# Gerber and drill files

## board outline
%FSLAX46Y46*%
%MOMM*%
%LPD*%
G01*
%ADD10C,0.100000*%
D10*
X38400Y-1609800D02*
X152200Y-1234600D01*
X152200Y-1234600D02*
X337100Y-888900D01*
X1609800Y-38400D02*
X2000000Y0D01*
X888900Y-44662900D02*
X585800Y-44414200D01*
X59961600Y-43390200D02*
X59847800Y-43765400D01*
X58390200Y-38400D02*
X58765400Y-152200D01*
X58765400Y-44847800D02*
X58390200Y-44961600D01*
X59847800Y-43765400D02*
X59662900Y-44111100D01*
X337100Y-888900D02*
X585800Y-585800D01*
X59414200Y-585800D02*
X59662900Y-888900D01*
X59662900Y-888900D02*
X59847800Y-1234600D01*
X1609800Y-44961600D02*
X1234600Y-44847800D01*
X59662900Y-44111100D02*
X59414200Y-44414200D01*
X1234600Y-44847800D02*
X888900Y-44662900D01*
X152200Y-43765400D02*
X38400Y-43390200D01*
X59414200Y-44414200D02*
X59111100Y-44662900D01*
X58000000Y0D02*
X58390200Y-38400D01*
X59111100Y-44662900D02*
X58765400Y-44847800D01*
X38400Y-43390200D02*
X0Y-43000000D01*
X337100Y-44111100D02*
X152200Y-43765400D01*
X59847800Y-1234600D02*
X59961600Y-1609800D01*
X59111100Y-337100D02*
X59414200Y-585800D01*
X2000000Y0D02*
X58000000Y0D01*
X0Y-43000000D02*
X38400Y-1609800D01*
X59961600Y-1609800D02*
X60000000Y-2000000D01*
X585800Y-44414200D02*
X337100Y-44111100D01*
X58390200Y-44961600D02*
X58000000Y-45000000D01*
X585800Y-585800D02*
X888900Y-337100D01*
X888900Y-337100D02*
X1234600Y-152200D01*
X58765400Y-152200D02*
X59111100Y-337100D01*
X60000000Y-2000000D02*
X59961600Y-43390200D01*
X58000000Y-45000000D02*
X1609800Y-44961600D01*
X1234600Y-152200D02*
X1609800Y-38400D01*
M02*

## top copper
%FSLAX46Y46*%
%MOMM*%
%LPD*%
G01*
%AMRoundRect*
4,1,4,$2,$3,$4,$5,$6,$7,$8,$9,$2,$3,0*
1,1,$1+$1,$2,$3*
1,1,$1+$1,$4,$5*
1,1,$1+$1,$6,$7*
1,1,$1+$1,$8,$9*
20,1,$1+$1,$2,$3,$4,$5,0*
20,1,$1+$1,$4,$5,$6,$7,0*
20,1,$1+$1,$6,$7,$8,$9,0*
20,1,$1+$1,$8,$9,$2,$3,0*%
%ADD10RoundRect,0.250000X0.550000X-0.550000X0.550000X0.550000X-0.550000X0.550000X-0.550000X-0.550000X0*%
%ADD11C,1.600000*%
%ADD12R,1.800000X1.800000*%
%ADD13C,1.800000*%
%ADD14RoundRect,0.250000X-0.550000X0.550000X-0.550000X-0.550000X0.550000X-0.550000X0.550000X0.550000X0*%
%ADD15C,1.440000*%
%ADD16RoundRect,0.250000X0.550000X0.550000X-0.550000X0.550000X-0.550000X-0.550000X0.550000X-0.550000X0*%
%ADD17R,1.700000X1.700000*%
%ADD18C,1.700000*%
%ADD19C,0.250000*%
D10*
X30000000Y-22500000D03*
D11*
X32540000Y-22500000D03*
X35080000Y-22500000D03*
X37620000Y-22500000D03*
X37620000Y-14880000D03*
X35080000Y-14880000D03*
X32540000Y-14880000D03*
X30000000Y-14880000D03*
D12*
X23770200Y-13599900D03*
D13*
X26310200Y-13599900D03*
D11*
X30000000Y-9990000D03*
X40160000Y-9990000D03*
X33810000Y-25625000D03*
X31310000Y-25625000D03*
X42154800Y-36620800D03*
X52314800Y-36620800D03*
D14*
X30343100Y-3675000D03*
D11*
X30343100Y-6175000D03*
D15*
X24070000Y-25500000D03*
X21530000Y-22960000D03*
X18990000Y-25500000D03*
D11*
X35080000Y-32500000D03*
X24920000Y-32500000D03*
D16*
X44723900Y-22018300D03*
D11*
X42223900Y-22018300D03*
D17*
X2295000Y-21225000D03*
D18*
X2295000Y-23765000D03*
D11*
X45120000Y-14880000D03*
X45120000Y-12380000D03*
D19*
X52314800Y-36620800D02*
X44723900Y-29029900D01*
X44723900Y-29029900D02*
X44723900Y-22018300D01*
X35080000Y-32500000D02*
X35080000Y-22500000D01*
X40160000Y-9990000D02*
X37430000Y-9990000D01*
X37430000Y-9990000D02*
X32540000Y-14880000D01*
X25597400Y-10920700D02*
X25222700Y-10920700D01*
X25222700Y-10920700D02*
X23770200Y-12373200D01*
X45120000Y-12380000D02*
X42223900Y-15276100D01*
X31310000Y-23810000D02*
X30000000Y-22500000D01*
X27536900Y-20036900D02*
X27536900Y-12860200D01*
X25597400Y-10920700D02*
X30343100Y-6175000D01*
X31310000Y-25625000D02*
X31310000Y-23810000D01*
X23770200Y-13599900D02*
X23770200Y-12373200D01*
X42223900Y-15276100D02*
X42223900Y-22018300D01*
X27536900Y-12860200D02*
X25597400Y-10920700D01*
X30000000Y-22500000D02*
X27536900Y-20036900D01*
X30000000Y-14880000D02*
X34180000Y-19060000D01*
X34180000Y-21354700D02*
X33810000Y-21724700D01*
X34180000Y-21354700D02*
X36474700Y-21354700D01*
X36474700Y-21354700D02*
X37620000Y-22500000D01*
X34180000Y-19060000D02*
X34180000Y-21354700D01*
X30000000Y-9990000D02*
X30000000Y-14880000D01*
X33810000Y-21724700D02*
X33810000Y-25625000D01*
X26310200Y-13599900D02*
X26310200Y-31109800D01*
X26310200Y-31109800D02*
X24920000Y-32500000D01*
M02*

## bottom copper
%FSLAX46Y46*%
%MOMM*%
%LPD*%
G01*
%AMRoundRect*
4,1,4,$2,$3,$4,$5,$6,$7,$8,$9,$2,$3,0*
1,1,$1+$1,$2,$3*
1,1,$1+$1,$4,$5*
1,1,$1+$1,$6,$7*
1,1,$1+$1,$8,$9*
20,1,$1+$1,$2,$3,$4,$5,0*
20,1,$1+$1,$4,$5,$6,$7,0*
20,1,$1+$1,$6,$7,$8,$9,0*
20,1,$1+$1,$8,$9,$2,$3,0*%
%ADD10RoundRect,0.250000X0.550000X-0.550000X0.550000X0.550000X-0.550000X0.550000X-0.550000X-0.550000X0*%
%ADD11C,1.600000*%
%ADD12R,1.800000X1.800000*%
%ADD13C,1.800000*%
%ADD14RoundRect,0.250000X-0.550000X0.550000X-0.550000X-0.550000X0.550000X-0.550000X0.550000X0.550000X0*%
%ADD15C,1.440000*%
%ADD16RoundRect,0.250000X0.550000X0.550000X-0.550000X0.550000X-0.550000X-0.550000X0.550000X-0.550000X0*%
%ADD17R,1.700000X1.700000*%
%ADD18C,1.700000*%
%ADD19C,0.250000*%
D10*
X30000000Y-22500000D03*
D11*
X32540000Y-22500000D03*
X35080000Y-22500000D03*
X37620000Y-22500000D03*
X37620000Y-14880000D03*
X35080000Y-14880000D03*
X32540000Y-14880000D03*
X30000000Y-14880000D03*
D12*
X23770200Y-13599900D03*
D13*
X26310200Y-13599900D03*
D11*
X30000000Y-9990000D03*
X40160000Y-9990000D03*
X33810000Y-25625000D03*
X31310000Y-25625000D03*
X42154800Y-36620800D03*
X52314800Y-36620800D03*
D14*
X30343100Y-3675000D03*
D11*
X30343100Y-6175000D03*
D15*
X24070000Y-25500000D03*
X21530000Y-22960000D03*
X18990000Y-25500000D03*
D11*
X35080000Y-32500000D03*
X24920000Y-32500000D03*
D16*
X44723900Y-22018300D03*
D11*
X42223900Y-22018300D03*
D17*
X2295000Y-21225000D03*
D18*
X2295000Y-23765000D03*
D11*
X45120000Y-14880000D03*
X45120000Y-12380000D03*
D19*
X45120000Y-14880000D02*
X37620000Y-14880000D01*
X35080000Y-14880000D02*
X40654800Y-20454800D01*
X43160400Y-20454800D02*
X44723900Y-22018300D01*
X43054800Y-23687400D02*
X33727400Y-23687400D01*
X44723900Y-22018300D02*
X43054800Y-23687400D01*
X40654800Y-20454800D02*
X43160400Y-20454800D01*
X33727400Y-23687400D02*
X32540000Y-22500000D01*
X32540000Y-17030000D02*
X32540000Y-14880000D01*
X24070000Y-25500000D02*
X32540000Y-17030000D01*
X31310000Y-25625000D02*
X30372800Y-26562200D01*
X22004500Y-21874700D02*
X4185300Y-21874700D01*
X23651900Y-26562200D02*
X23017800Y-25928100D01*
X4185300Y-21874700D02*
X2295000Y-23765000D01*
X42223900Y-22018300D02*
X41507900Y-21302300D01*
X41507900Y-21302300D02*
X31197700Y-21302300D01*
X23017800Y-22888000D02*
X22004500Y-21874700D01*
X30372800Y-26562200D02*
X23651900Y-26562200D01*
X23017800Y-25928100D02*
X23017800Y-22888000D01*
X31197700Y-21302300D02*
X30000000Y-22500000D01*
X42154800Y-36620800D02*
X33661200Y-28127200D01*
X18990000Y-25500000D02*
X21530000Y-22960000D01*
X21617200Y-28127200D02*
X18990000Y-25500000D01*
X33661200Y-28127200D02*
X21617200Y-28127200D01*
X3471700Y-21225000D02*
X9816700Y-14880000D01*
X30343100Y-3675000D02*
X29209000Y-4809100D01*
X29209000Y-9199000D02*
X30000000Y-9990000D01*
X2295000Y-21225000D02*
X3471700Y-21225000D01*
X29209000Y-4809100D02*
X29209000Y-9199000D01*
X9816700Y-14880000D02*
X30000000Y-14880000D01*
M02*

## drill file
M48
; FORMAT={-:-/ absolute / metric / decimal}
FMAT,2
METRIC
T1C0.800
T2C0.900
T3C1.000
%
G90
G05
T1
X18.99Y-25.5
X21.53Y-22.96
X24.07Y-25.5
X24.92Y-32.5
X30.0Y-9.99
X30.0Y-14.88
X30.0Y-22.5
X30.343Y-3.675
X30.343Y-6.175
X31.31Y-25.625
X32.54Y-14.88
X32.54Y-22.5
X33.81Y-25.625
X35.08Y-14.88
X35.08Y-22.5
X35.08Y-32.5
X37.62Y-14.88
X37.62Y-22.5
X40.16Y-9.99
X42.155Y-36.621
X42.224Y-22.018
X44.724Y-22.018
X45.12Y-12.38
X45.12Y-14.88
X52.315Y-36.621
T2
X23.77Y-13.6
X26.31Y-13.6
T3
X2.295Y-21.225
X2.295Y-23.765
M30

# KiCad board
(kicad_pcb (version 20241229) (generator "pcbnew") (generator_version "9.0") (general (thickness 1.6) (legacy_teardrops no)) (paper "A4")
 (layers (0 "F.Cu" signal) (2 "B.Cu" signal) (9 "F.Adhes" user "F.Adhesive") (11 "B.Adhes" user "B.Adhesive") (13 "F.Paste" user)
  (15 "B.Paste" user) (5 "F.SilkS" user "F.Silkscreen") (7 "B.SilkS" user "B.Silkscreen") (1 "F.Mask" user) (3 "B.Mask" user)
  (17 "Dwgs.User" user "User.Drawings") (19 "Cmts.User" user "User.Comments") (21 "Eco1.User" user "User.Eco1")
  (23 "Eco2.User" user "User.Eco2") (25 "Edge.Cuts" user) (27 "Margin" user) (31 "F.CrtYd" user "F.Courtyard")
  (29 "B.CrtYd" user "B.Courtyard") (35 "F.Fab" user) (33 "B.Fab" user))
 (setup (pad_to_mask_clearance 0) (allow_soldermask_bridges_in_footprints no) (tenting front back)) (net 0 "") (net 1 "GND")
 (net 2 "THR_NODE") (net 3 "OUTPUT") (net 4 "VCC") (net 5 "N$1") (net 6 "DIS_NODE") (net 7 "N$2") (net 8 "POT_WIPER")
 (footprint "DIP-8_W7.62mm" (layer "F.Cu") (at 30 22.5 90)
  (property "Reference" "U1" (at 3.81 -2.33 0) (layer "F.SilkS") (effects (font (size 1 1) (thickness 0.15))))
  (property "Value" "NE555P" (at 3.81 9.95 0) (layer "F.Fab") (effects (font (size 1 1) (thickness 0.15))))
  (pad "1" thru_hole roundrect (at 0 0 90) (size 1.6 1.6) (drill 0.8) (layers "*.Cu" "*.Mask") (remove_unused_layers no)
   (roundrect_rratio 0.15625) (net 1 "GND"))
  (pad "2" thru_hole circle (at 0 2.54 90) (size 1.6 1.6) (drill 0.8) (layers "*.Cu" "*.Mask") (remove_unused_layers no) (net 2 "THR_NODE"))
  (pad "3" thru_hole circle (at 0 5.08 90) (size 1.6 1.6) (drill 0.8) (layers "*.Cu" "*.Mask") (remove_unused_layers no) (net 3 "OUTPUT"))
  (pad "4" thru_hole circle (at 0 7.62 90) (size 1.6 1.6) (drill 0.8) (layers "*.Cu" "*.Mask") (remove_unused_layers no) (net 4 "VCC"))
  (pad "5" thru_hole circle (at 7.62 7.62 90) (size 1.6 1.6) (drill 0.8) (layers "*.Cu" "*.Mask") (remove_unused_layers no) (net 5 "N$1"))
  (pad "6" thru_hole circle (at 7.62 5.08 90) (size 1.6 1.6) (drill 0.8) (layers "*.Cu" "*.Mask") (remove_unused_layers no)
   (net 2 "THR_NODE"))
  (pad "7" thru_hole circle (at 7.62 2.54 90) (size 1.6 1.6) (drill 0.8) (layers "*.Cu" "*.Mask") (remove_unused_layers no)
   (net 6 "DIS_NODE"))
  (pad "8" thru_hole circle (at 7.62 0 90) (size 1.6 1.6) (drill 0.8) (layers "*.Cu" "*.Mask") (remove_unused_layers no) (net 4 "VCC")))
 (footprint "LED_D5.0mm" (layer "F.Cu") (at 23.7702 13.5999)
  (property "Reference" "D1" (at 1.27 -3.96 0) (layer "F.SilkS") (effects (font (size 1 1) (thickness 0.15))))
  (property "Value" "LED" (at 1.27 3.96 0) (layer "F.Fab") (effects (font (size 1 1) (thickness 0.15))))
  (pad "1" thru_hole rect (at 0 0) (size 1.8 1.8) (drill 0.9) (layers "*.Cu" "*.Mask") (remove_unused_layers no) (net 1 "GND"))
  (pad "2" thru_hole circle (at 2.54 0) (size 1.8 1.8) (drill 0.9) (layers "*.Cu" "*.Mask") (remove_unused_layers no) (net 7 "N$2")))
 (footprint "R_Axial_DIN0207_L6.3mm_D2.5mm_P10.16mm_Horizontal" (layer "F.Cu") (at 30 9.99)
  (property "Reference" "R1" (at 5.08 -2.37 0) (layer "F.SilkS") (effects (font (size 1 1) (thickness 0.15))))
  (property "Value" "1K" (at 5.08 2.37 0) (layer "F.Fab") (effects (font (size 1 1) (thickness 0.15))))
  (pad "1" thru_hole circle (at 0 0) (size 1.6 1.6) (drill 0.8) (layers "*.Cu" "*.Mask") (remove_unused_layers no) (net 4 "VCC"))
  (pad "2" thru_hole circle (at 10.16 0) (size 1.6 1.6) (drill 0.8) (layers "*.Cu" "*.Mask") (remove_unused_layers no) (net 6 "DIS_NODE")))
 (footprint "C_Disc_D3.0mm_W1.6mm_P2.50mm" (layer "F.Cu") (at 33.81 25.625 180)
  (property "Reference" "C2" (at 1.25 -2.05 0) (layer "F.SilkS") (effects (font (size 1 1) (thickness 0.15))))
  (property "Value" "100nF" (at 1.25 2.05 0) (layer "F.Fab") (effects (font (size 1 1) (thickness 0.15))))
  (pad "1" thru_hole circle (at 0 0 180) (size 1.6 1.6) (drill 0.8) (layers "*.Cu" "*.Mask") (remove_unused_layers no) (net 4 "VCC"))
  (pad "2" thru_hole circle (at 2.5 0 180) (size 1.6 1.6) (drill 0.8) (layers "*.Cu" "*.Mask") (remove_unused_layers no) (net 1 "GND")))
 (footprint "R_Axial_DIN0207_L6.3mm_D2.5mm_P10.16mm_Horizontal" (layer "F.Cu") (at 42.1548 36.6208)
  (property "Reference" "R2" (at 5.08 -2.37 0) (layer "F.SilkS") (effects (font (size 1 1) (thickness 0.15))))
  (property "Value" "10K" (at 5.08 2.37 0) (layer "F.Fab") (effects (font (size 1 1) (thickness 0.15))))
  (pad "1" thru_hole circle (at 0 0) (size 1.6 1.6) (drill 0.8) (layers "*.Cu" "*.Mask") (remove_unused_layers no) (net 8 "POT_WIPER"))
  (pad "2" thru_hole circle (at 10.16 0) (size 1.6 1.6) (drill 0.8) (layers "*.Cu" "*.Mask") (remove_unused_layers no) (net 2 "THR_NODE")))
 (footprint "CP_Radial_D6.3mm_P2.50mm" (layer "F.Cu") (at 30.3431 3.675 -90)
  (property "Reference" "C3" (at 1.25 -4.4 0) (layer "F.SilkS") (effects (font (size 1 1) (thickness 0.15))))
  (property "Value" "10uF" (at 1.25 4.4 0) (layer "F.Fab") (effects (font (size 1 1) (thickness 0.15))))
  (pad "1" thru_hole roundrect (at 0 0 270) (size 1.6 1.6) (drill 0.8) (layers "*.Cu" "*.Mask") (remove_unused_layers no)
   (roundrect_rratio 0.15625) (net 4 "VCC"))
  (pad "2" thru_hole circle (at 2.5 0 270) (size 1.6 1.6) (drill 0.8) (layers "*.Cu" "*.Mask") (remove_unused_layers no) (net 1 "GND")))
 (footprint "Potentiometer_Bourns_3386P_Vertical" (layer "F.Cu") (at 24.07 25.5 90)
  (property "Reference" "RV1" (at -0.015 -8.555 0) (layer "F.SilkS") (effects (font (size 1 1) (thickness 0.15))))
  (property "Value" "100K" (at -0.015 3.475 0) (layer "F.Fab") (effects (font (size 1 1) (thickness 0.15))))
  (pad "1" thru_hole circle (at 0 0 90) (size 1.44 1.44) (drill 0.8) (layers "*.Cu" "*.Mask") (remove_unused_layers no) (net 6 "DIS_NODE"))
  (pad "2" thru_hole circle (at 2.54 -2.54 90) (size 1.44 1.44) (drill 0.8) (layers "*.Cu" "*.Mask") (remove_unused_layers no)
   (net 8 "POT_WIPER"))
  (pad "3" thru_hole circle (at 0 -5.08 90) (size 1.44 1.44) (drill 0.8) (layers "*.Cu" "*.Mask") (remove_unused_layers no)
   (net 8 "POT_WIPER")))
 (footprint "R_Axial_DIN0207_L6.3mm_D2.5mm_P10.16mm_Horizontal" (layer "F.Cu") (at 35.08 32.5 180)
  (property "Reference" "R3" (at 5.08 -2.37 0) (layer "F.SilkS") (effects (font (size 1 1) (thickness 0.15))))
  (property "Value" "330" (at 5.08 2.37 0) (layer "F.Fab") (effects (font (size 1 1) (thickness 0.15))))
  (pad "1" thru_hole circle (at 0 0 180) (size 1.6 1.6) (drill 0.8) (layers "*.Cu" "*.Mask") (remove_unused_layers no) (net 3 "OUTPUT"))
  (pad "2" thru_hole circle (at 10.16 0 180) (size 1.6 1.6) (drill 0.8) (layers "*.Cu" "*.Mask") (remove_unused_layers no) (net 7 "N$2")))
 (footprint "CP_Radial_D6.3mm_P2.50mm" (layer "F.Cu") (at 44.7239 22.0183 180)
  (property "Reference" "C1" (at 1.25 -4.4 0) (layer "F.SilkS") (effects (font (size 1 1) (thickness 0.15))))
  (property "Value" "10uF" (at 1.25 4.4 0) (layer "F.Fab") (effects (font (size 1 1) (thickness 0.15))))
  (pad "1" thru_hole roundrect (at 0 0 180) (size 1.6 1.6) (drill 0.8) (layers "*.Cu" "*.Mask") (remove_unused_layers no)
   (roundrect_rratio 0.15625) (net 2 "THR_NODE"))
  (pad "2" thru_hole circle (at 2.5 0 180) (size 1.6 1.6) (drill 0.8) (layers "*.Cu" "*.Mask") (remove_unused_layers no) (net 1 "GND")))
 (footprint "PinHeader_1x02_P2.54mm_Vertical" (layer "F.Cu") (at 2.295 21.225)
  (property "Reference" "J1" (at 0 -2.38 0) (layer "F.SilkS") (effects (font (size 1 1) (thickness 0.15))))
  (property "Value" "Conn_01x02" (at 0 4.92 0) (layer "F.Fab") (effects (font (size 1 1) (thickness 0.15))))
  (pad "1" thru_hole rect (at 0 0) (size 1.7 1.7) (drill 1) (layers "*.Cu" "*.Mask") (remove_unused_layers no) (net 4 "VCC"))
  (pad "2" thru_hole circle (at 0 2.54) (size 1.7 1.7) (drill 1) (layers "*.Cu" "*.Mask") (remove_unused_layers no) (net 1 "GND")))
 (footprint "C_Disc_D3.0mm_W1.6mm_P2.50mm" (layer "F.Cu") (at 45.12 14.88 90)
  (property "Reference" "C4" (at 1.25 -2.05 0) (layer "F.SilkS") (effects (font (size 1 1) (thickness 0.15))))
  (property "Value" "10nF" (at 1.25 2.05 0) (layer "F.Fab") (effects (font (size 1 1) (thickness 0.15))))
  (pad "1" thru_hole circle (at 0 0 90) (size 1.6 1.6) (drill 0.8) (layers "*.Cu" "*.Mask") (remove_unused_layers no) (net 5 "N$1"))
  (pad "2" thru_hole circle (at 2.5 0 90) (size 1.6 1.6) (drill 0.8) (layers "*.Cu" "*.Mask") (remove_unused_layers no) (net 1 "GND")))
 (gr_line (start 0.0384 1.6098) (end 0.1522 1.2346) (stroke (width 0.1) (type solid)) (layer "Edge.Cuts"))
 (gr_line (start 0.1522 1.2346) (end 0.3371 0.8889) (stroke (width 0.1) (type solid)) (layer "Edge.Cuts"))
 (gr_line (start 1.6098 0.0384) (end 2 0) (stroke (width 0.1) (type solid)) (layer "Edge.Cuts"))
 (gr_line (start 0.8889 44.6629) (end 0.5858 44.4142) (stroke (width 0.1) (type solid)) (layer "Edge.Cuts"))
 (gr_line (start 59.9616 43.3902) (end 59.8478 43.7654) (stroke (width 0.1) (type solid)) (layer "Edge.Cuts"))
 (gr_line (start 58.3902 0.0384) (end 58.7654 0.1522) (stroke (width 0.1) (type solid)) (layer "Edge.Cuts"))
 (gr_line (start 58.7654 44.8478) (end 58.3902 44.9616) (stroke (width 0.1) (type solid)) (layer "Edge.Cuts"))
 (gr_line (start 59.8478 43.7654) (end 59.6629 44.1111) (stroke (width 0.1) (type solid)) (layer "Edge.Cuts"))
 (gr_line (start 0.3371 0.8889) (end 0.5858 0.5858) (stroke (width 0.1) (type solid)) (layer "Edge.Cuts"))
 (gr_line (start 59.4142 0.5858) (end 59.6629 0.8889) (stroke (width 0.1) (type solid)) (layer "Edge.Cuts"))
 (gr_line (start 59.6629 0.8889) (end 59.8478 1.2346) (stroke (width 0.1) (type solid)) (layer "Edge.Cuts"))
 (gr_line (start 1.6098 44.9616) (end 1.2346 44.8478) (stroke (width 0.1) (type solid)) (layer "Edge.Cuts"))
 (gr_line (start 59.6629 44.1111) (end 59.4142 44.4142) (stroke (width 0.1) (type solid)) (layer "Edge.Cuts"))
 (gr_line (start 1.2346 44.8478) (end 0.8889 44.6629) (stroke (width 0.1) (type solid)) (layer "Edge.Cuts"))
 (gr_line (start 0.1522 43.7654) (end 0.0384 43.3902) (stroke (width 0.1) (type solid)) (layer "Edge.Cuts"))
 (gr_line (start 59.4142 44.4142) (end 59.1111 44.6629) (stroke (width 0.1) (type solid)) (layer "Edge.Cuts"))
 (gr_line (start 58 0) (end 58.3902 0.0384) (stroke (width 0.1) (type solid)) (layer "Edge.Cuts"))
 (gr_line (start 59.1111 44.6629) (end 58.7654 44.8478) (stroke (width 0.1) (type solid)) (layer "Edge.Cuts"))
 (gr_line (start 0.0384 43.3902) (end 0 43) (stroke (width 0.1) (type solid)) (layer "Edge.Cuts"))
 (gr_line (start 0.3371 44.1111) (end 0.1522 43.7654) (stroke (width 0.1) (type solid)) (layer "Edge.Cuts"))
 (gr_line (start 59.8478 1.2346) (end 59.9616 1.6098) (stroke (width 0.1) (type solid)) (layer "Edge.Cuts"))
 (gr_line (start 59.1111 0.3371) (end 59.4142 0.5858) (stroke (width 0.1) (type solid)) (layer "Edge.Cuts"))
 (gr_line (start 2 0) (end 58 0) (stroke (width 0.1) (type solid)) (layer "Edge.Cuts"))
 (gr_line (start 0 43) (end 0.0384 1.6098) (stroke (width 0.1) (type solid)) (layer "Edge.Cuts"))
 (gr_line (start 59.9616 1.6098) (end 60 2) (stroke (width 0.1) (type solid)) (layer "Edge.Cuts"))
 (gr_line (start 0.5858 44.4142) (end 0.3371 44.1111) (stroke (width 0.1) (type solid)) (layer "Edge.Cuts"))
 (gr_line (start 58.3902 44.9616) (end 58 45) (stroke (width 0.1) (type solid)) (layer "Edge.Cuts"))
 (gr_line (start 0.5858 0.5858) (end 0.8889 0.3371) (stroke (width 0.1) (type solid)) (layer "Edge.Cuts"))
 (gr_line (start 0.8889 0.3371) (end 1.2346 0.1522) (stroke (width 0.1) (type solid)) (layer "Edge.Cuts"))
 (gr_line (start 58.7654 0.1522) (end 59.1111 0.3371) (stroke (width 0.1) (type solid)) (layer "Edge.Cuts"))
 (gr_line (start 60 2) (end 59.9616 43.3902) (stroke (width 0.1) (type solid)) (layer "Edge.Cuts"))
 (gr_line (start 58 45) (end 1.6098 44.9616) (stroke (width 0.1) (type solid)) (layer "Edge.Cuts"))
 (gr_line (start 1.2346 0.1522) (end 1.6098 0.0384) (stroke (width 0.1) (type solid)) (layer "Edge.Cuts"))
 (segment (start 45.12 14.88) (end 37.62 14.88) (width 0.25) (layer "B.Cu") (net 5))
 (segment (start 52.3148 36.6208) (end 44.7239 29.0299) (width 0.25) (layer "F.Cu") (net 2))
 (segment (start 44.7239 29.0299) (end 44.7239 22.0183) (width 0.25) (layer "F.Cu") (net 2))
 (segment (start 35.08 14.88) (end 40.6548 20.4548) (width 0.25) (layer "B.Cu") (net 2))
 (segment (start 43.1604 20.4548) (end 44.7239 22.0183) (width 0.25) (layer "B.Cu") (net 2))
 (segment (start 43.0548 23.6874) (end 33.7274 23.6874) (width 0.25) (layer "B.Cu") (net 2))
 (segment (start 44.7239 22.0183) (end 43.0548 23.6874) (width 0.25) (layer "B.Cu") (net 2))
 (segment (start 40.6548 20.4548) (end 43.1604 20.4548) (width 0.25) (layer "B.Cu") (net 2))
 (segment (start 33.7274 23.6874) (end 32.54 22.5) (width 0.25) (layer "B.Cu") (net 2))
 (segment (start 35.08 32.5) (end 35.08 22.5) (width 0.25) (layer "F.Cu") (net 3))
 (segment (start 40.16 9.99) (end 37.43 9.99) (width 0.25) (layer "F.Cu") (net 6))
 (segment (start 37.43 9.99) (end 32.54 14.88) (width 0.25) (layer "F.Cu") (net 6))
 (segment (start 32.54 17.03) (end 32.54 14.88) (width 0.25) (layer "B.Cu") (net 6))
 (segment (start 24.07 25.5) (end 32.54 17.03) (width 0.25) (layer "B.Cu") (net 6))
 (segment (start 25.5974 10.9207) (end 25.2227 10.9207) (width 0.25) (layer "F.Cu") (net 1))
 (segment (start 25.2227 10.9207) (end 23.7702 12.3732) (width 0.25) (layer "F.Cu") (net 1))
 (segment (start 45.12 12.38) (end 42.2239 15.2761) (width 0.25) (layer "F.Cu") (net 1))
 (segment (start 31.31 23.81) (end 30 22.5) (width 0.25) (layer "F.Cu") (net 1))
 (segment (start 27.5369 20.0369) (end 27.5369 12.8602) (width 0.25) (layer "F.Cu") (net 1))
 (segment (start 25.5974 10.9207) (end 30.3431 6.175) (width 0.25) (layer "F.Cu") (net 1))
 (segment (start 31.31 25.625) (end 31.31 23.81) (width 0.25) (layer "F.Cu") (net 1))
 (segment (start 23.7702 13.5999) (end 23.7702 12.3732) (width 0.25) (layer "F.Cu") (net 1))
 (segment (start 42.2239 15.2761) (end 42.2239 22.0183) (width 0.25) (layer "F.Cu") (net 1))
 (segment (start 27.5369 12.8602) (end 25.5974 10.9207) (width 0.25) (layer "F.Cu") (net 1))
 (segment (start 30 22.5) (end 27.5369 20.0369) (width 0.25) (layer "F.Cu") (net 1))
 (segment (start 31.31 25.625) (end 30.3728 26.5622) (width 0.25) (layer "B.Cu") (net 1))
 (segment (start 22.0045 21.8747) (end 4.1853 21.8747) (width 0.25) (layer "B.Cu") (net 1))
 (segment (start 23.6519 26.5622) (end 23.0178 25.9281) (width 0.25) (layer "B.Cu") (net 1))
 (segment (start 4.1853 21.8747) (end 2.295 23.765) (width 0.25) (layer "B.Cu") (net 1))
 (segment (start 42.2239 22.0183) (end 41.5079 21.3023) (width 0.25) (layer "B.Cu") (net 1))
 (segment (start 41.5079 21.3023) (end 31.1977 21.3023) (width 0.25) (layer "B.Cu") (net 1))
 (segment (start 23.0178 22.888) (end 22.0045 21.8747) (width 0.25) (layer "B.Cu") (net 1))
 (segment (start 30.3728 26.5622) (end 23.6519 26.5622) (width 0.25) (layer "B.Cu") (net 1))
 (segment (start 23.0178 25.9281) (end 23.0178 22.888) (width 0.25) (layer "B.Cu") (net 1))
 (segment (start 31.1977 21.3023) (end 30 22.5) (width 0.25) (layer "B.Cu") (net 1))
 (segment (start 42.1548 36.6208) (end 33.6612 28.1272) (width 0.25) (layer "B.Cu") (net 8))
 (segment (start 18.99 25.5) (end 21.53 22.96) (width 0.25) (layer "B.Cu") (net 8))
 (segment (start 21.6172 28.1272) (end 18.99 25.5) (width 0.25) (layer "B.Cu") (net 8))
 (segment (start 33.6612 28.1272) (end 21.6172 28.1272) (width 0.25) (layer "B.Cu") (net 8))
 (segment (start 30 14.88) (end 34.18 19.06) (width 0.25) (layer "F.Cu") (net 4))
 (segment (start 34.18 21.3547) (end 33.81 21.7247) (width 0.25) (layer "F.Cu") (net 4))
 (segment (start 34.18 21.3547) (end 36.4747 21.3547) (width 0.25) (layer "F.Cu") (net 4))
 (segment (start 36.4747 21.3547) (end 37.62 22.5) (width 0.25) (layer "F.Cu") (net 4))
 (segment (start 34.18 19.06) (end 34.18 21.3547) (width 0.25) (layer "F.Cu") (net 4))
 (segment (start 30 9.99) (end 30 14.88) (width 0.25) (layer "F.Cu") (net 4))
 (segment (start 33.81 21.7247) (end 33.81 25.625) (width 0.25) (layer "F.Cu") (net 4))
 (segment (start 3.4717 21.225) (end 9.8167 14.88) (width 0.25) (layer "B.Cu") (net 4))
 (segment (start 30.3431 3.675) (end 29.209 4.8091) (width 0.25) (layer "B.Cu") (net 4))
 (segment (start 29.209 9.199) (end 30 9.99) (width 0.25) (layer "B.Cu") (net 4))
 (segment (start 2.295 21.225) (end 3.4717 21.225) (width 0.25) (layer "B.Cu") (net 4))
 (segment (start 29.209 4.8091) (end 29.209 9.199) (width 0.25) (layer "B.Cu") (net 4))
 (segment (start 9.8167 14.88) (end 30 14.88) (width 0.25) (layer "B.Cu") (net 4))
 (segment (start 26.3102 13.5999) (end 26.3102 31.1098) (width 0.25) (layer "F.Cu") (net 7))
 (segment (start 26.3102 31.1098) (end 24.92 32.5) (width 0.25) (layer "F.Cu") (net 7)))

